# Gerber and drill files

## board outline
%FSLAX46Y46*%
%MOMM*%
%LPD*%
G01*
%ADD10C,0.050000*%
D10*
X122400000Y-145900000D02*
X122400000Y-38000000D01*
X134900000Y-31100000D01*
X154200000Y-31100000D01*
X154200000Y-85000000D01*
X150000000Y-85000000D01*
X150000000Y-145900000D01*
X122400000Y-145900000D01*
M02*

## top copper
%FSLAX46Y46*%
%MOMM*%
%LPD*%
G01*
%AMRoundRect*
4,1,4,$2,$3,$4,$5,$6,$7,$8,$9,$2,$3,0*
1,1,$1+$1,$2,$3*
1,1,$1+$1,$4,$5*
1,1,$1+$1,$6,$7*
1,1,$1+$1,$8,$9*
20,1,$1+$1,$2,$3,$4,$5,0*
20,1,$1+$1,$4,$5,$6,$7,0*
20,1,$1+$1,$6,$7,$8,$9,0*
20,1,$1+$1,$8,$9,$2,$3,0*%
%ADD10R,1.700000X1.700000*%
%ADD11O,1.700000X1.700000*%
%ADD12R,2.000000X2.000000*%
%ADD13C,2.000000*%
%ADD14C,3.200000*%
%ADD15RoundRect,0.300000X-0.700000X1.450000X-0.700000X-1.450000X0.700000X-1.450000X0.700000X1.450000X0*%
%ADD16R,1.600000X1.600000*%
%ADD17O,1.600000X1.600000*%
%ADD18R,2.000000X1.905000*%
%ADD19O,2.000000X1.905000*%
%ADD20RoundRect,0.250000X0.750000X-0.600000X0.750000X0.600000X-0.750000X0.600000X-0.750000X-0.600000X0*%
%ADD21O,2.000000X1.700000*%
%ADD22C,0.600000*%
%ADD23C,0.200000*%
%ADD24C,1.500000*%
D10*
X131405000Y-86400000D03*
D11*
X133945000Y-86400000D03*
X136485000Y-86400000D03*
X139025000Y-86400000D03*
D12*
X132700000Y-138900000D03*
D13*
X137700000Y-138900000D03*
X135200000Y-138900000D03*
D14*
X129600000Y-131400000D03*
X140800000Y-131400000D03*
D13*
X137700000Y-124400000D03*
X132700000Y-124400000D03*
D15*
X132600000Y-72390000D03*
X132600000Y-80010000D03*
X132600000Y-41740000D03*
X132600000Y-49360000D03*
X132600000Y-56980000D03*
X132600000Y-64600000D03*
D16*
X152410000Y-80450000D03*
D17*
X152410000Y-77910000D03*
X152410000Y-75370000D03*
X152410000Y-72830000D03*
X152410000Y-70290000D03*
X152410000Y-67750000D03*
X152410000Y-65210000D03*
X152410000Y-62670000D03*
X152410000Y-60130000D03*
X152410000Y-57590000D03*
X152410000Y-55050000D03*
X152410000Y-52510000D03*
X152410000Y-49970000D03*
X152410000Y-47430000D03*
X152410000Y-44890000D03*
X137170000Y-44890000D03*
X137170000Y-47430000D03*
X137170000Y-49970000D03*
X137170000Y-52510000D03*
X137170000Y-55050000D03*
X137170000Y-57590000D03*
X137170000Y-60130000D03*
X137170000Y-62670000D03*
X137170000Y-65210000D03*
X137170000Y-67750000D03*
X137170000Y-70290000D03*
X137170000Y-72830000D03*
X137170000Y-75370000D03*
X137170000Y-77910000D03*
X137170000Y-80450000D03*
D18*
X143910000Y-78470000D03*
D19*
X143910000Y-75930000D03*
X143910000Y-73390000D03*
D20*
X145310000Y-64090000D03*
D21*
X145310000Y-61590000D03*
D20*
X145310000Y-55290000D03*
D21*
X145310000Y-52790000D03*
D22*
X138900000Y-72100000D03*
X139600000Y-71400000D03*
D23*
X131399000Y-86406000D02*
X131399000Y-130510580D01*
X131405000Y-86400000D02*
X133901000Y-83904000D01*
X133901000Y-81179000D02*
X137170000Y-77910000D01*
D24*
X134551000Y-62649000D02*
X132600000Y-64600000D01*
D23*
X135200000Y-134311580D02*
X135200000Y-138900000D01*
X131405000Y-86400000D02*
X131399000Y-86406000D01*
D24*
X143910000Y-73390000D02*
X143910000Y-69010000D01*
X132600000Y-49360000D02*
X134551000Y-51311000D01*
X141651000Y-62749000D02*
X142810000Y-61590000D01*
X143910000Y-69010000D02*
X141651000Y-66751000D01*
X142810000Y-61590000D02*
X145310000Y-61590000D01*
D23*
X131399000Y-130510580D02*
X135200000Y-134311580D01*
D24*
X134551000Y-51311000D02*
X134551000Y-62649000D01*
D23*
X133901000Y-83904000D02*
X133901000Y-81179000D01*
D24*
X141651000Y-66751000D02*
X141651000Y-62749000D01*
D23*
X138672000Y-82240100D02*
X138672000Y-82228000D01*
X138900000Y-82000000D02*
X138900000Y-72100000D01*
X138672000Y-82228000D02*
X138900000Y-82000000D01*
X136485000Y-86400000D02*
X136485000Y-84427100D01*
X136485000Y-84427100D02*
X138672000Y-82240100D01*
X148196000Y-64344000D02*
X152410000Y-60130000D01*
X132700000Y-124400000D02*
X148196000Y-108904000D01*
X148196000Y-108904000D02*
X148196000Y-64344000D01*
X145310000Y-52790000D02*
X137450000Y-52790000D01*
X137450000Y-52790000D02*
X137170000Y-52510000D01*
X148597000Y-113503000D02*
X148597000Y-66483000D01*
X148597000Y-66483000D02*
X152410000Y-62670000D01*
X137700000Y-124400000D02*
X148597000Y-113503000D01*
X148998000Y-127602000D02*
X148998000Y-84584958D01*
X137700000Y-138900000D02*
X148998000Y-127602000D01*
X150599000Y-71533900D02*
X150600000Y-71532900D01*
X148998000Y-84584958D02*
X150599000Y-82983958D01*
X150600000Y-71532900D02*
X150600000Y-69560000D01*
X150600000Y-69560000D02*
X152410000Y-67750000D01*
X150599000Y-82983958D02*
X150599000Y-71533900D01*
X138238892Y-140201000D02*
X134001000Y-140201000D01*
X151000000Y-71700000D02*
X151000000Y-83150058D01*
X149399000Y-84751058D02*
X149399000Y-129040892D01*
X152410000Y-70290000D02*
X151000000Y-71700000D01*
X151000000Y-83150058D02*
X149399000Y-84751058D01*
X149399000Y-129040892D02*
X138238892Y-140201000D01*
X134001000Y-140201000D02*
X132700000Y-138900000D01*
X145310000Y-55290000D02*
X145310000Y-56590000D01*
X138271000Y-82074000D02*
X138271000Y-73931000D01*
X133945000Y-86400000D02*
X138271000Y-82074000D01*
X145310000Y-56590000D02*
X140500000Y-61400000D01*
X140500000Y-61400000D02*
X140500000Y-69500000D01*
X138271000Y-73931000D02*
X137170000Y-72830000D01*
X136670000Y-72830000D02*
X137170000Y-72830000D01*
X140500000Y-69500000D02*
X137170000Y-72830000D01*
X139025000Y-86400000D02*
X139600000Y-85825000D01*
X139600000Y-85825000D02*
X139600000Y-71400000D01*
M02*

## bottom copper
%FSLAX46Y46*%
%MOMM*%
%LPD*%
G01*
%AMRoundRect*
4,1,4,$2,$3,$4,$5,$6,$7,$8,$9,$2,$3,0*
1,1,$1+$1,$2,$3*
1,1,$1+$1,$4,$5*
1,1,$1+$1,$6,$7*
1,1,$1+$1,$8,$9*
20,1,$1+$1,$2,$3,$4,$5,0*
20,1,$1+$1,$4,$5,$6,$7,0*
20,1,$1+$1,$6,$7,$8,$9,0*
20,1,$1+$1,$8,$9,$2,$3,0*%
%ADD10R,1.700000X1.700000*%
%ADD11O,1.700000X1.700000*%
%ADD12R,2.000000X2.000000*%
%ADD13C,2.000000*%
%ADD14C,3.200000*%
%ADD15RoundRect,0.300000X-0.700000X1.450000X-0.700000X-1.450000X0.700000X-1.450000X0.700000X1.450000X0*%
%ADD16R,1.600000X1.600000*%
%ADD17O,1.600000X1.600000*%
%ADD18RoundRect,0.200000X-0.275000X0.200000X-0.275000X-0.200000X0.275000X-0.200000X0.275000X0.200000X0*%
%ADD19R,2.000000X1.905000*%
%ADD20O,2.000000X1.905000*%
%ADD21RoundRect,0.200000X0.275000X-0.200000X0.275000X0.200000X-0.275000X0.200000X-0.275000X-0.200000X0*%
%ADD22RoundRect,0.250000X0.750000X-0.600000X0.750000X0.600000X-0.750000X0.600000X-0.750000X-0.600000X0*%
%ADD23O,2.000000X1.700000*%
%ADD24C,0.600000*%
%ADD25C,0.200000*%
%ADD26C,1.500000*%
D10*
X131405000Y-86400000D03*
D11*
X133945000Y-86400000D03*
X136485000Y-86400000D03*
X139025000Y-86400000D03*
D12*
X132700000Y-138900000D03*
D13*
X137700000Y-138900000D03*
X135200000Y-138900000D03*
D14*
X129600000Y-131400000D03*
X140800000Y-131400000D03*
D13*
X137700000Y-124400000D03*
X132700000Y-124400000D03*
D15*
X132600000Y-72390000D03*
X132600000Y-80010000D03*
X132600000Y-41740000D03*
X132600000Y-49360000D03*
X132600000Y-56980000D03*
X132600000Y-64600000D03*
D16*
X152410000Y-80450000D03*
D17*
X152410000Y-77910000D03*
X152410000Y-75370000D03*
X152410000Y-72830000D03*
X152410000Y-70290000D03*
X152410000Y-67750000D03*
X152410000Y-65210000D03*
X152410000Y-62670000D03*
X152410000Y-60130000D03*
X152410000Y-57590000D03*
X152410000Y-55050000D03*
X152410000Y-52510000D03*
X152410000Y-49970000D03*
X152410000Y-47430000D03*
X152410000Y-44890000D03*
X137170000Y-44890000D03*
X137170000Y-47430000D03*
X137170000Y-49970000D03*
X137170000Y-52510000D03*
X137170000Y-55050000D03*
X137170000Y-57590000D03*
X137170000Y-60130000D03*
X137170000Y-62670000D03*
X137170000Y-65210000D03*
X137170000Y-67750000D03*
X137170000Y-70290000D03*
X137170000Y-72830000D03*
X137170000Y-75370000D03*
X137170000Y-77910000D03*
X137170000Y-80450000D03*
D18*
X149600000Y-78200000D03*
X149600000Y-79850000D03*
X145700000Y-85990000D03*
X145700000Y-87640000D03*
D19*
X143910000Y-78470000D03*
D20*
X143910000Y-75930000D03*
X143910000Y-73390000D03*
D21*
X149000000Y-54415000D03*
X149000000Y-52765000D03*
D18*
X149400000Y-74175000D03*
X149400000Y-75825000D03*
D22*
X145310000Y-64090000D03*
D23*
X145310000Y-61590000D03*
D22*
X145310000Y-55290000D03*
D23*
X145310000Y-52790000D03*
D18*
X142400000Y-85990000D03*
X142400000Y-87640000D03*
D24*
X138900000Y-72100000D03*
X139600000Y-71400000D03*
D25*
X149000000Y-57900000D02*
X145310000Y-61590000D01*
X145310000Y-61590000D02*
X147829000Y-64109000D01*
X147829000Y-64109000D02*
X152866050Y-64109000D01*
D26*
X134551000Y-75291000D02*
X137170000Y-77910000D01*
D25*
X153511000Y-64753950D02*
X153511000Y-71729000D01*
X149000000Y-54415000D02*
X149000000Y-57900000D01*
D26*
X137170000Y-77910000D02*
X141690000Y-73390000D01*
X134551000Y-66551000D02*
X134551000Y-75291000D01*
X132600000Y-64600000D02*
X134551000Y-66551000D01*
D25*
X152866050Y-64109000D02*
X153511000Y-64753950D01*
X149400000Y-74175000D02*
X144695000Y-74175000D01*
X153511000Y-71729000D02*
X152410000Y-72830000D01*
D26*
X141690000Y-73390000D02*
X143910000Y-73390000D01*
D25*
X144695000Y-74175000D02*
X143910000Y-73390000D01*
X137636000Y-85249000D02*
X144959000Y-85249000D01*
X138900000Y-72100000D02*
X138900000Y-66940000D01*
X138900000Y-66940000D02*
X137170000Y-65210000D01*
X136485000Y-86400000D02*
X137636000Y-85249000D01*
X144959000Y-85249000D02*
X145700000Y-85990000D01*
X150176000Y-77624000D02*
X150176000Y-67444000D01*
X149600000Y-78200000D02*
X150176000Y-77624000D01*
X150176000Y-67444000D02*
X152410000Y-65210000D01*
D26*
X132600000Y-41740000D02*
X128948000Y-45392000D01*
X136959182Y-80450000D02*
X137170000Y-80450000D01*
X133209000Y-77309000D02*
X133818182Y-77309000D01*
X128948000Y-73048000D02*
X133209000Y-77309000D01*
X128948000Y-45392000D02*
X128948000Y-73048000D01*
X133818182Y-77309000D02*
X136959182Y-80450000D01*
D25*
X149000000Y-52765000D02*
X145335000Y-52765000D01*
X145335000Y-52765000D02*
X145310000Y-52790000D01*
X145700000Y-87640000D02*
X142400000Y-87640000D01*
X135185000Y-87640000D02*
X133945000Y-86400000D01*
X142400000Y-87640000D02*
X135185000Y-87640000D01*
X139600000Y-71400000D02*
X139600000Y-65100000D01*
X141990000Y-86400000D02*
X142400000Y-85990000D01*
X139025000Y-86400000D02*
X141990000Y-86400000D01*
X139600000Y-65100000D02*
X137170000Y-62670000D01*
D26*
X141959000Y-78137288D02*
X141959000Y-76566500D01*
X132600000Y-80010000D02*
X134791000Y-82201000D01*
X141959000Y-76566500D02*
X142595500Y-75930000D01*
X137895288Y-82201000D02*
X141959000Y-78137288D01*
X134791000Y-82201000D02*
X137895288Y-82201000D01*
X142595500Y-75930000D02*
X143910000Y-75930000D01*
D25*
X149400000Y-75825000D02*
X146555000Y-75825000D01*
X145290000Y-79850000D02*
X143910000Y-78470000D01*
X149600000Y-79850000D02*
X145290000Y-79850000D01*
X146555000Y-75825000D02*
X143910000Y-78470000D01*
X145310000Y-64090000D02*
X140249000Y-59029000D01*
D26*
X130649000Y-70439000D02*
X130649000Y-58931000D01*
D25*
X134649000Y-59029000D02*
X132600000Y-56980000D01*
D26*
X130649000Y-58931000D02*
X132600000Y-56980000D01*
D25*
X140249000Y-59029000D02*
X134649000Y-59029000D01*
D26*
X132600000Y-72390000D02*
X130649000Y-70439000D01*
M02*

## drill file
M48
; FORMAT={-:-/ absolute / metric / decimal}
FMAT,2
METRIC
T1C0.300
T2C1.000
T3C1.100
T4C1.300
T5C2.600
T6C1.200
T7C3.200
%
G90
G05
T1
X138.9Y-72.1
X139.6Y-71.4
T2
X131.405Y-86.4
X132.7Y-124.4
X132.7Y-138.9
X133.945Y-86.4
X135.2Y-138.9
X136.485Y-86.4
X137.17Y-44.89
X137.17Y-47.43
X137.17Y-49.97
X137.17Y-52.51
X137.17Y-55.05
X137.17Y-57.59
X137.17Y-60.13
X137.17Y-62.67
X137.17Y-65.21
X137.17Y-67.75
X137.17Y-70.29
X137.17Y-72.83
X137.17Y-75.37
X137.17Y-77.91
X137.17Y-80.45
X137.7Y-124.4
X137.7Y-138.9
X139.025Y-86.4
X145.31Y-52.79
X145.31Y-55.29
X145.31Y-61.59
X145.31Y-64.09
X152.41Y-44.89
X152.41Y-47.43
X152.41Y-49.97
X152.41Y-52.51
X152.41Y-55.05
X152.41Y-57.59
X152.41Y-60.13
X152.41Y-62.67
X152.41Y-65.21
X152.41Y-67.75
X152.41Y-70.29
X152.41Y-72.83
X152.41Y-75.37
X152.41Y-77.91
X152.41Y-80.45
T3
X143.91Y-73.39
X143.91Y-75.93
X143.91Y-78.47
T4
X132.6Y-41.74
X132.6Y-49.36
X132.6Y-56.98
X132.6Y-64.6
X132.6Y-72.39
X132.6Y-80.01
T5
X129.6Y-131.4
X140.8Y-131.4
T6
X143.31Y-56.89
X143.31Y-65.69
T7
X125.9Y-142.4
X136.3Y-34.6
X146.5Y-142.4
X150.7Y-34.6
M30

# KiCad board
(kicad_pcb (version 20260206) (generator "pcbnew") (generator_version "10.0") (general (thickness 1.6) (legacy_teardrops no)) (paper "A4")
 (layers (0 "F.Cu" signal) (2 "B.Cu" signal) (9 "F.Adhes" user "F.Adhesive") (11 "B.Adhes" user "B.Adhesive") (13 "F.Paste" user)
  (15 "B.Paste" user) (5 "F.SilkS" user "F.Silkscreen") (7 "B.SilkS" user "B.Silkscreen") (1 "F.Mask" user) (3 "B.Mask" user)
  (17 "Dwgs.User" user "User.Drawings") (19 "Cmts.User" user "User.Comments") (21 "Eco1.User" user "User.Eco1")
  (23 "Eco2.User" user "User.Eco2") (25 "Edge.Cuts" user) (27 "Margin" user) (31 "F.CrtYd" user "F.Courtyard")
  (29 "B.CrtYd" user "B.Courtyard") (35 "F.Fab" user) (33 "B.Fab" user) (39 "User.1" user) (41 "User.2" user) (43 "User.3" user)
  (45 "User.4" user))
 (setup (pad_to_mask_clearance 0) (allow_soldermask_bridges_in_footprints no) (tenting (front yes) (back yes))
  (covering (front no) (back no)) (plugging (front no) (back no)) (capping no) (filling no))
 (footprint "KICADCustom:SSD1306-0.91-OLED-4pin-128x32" (layer "F.Cu") (at 129.215 122.9 90)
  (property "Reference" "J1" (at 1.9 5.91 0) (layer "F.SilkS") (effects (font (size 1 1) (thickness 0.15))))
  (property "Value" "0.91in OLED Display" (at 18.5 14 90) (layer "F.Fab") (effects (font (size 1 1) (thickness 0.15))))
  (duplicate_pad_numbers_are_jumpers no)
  (pad "1" thru_hole rect (at 36.5 2.19 90) (size 1.7 1.7) (drill 1) (layers "*.Cu" "*.Mask") (remove_unused_layers no) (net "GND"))
  (pad "2" thru_hole oval (at 36.5 4.73 90) (size 1.7 1.7) (drill 1) (layers "*.Cu" "*.Mask") (remove_unused_layers no) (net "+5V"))
  (pad "3" thru_hole oval (at 36.5 7.27 90) (size 1.7 1.7) (drill 1) (layers "*.Cu" "*.Mask") (remove_unused_layers no) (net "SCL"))
  (pad "4" thru_hole oval (at 36.5 9.81 90) (size 1.7 1.7) (drill 1) (layers "*.Cu" "*.Mask") (remove_unused_layers no) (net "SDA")))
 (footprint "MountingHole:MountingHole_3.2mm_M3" (layer "F.Cu") (at 146.5 142.4)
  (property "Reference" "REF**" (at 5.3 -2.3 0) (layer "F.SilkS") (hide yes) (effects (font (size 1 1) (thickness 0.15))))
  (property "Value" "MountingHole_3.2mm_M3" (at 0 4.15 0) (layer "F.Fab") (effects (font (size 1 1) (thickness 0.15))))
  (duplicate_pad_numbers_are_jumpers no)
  (pad "" np_thru_hole circle (at 0 0) (size 3.2 3.2) (drill 3.2) (layers "*.Cu" "*.Mask")))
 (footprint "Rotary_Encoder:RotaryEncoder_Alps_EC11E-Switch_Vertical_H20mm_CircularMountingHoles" (layer "F.Cu") (at 132.7 138.9 90)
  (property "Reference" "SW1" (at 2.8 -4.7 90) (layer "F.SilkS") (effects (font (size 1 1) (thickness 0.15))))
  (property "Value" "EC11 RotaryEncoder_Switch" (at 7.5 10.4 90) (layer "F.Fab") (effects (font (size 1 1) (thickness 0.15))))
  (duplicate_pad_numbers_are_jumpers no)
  (pad "A" thru_hole rect (at 0 0 90) (size 2 2) (drill 1) (layers "*.Cu" "*.Mask") (remove_unused_layers no) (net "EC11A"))
  (pad "B" thru_hole circle (at 0 5 90) (size 2 2) (drill 1) (layers "*.Cu" "*.Mask") (remove_unused_layers no) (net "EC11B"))
  (pad "C" thru_hole circle (at 0 2.5 90) (size 2 2) (drill 1) (layers "*.Cu" "*.Mask") (remove_unused_layers no) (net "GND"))
  (pad "MP" thru_hole circle (at 7.5 -3.1 90) (size 3.2 3.2) (drill 2.6) (layers "*.Cu" "*.Mask") (remove_unused_layers no))
  (pad "MP" thru_hole circle (at 7.5 8.1 90) (size 3.2 3.2) (drill 2.6) (layers "*.Cu" "*.Mask") (remove_unused_layers no))
  (pad "S1" thru_hole circle (at 14.5 5 90) (size 2 2) (drill 1) (layers "*.Cu" "*.Mask") (remove_unused_layers no) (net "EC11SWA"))
  (pad "S2" thru_hole circle (at 14.5 0 90) (size 2 2) (drill 1) (layers "*.Cu" "*.Mask") (remove_unused_layers no) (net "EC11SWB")))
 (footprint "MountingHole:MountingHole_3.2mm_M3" (layer "F.Cu") (at 136.3 34.6)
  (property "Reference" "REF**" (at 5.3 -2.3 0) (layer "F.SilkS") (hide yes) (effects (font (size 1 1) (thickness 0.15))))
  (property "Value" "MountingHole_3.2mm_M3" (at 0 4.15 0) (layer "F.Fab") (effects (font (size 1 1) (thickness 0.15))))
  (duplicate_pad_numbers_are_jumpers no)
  (pad "" np_thru_hole circle (at 0 0) (size 3.2 3.2) (drill 3.2) (layers "*.Cu" "*.Mask")))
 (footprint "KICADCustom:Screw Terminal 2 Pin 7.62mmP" (layer "F.Cu") (at 132.6 72.39 -90)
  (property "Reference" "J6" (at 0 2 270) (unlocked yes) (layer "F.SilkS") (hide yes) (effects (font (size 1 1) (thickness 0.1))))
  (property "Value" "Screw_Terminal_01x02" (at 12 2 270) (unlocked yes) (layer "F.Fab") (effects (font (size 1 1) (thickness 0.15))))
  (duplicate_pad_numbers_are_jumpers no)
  (pad "1" thru_hole roundrect (at 0 0 270) (size 3.5 2) (drill 1.3) (layers "*.Cu" "*.Mask") (remove_unused_layers no)
   (roundrect_rratio 0.15) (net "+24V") (thermal_bridge_angle 45))
  (pad "2" thru_hole roundrect (at 7.62 0 270) (size 3.5 2) (drill 1.3) (layers "*.Cu" "*.Mask") (remove_unused_layers no)
   (roundrect_rratio 0.15) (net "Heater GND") (thermal_bridge_angle 45)))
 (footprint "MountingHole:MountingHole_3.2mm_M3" (layer "F.Cu") (at 150.7 34.6)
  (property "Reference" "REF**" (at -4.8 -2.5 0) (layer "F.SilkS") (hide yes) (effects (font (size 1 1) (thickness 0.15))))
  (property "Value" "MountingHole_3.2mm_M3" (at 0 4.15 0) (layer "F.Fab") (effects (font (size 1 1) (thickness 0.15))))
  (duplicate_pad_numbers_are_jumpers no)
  (pad "" np_thru_hole circle (at 0 0) (size 3.2 3.2) (drill 3.2) (layers "*.Cu" "*.Mask")))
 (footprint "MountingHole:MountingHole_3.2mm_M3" (layer "F.Cu") (at 125.9 142.4)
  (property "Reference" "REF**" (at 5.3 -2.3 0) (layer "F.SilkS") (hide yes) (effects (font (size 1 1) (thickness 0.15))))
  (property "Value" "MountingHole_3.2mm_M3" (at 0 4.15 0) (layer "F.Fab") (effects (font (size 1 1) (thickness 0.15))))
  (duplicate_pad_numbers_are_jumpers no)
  (pad "" np_thru_hole circle (at 0 0) (size 3.2 3.2) (drill 3.2) (layers "*.Cu" "*.Mask")))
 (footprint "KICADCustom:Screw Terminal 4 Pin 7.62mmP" (layer "F.Cu") (at 132.6 41.74 -90)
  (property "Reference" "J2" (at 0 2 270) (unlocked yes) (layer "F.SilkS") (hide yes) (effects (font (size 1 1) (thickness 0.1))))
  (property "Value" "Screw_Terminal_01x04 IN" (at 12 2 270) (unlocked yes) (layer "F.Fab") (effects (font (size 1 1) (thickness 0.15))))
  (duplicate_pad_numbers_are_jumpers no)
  (pad "1" thru_hole roundrect (at 0 0 270) (size 3.5 2) (drill 1.3) (layers "*.Cu" "*.Mask") (remove_unused_layers no)
   (roundrect_rratio 0.15) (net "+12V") (thermal_bridge_angle 45))
  (pad "2" thru_hole roundrect (at 7.62 0 270) (size 3.5 2) (drill 1.3) (layers "*.Cu" "*.Mask") (remove_unused_layers no)
   (roundrect_rratio 0.15) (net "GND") (thermal_bridge_angle 45))
  (pad "3" thru_hole roundrect (at 15.24 0 270) (size 3.5 2) (drill 1.3) (layers "*.Cu" "*.Mask") (remove_unused_layers no)
   (roundrect_rratio 0.15) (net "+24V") (thermal_bridge_angle 45))
  (pad "4" thru_hole roundrect (at 22.86 0 270) (size 3.5 2) (drill 1.3) (layers "*.Cu" "*.Mask") (remove_unused_layers no)
   (roundrect_rratio 0.15) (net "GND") (thermal_bridge_angle 45)))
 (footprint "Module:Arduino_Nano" (layer "F.Cu") (at 152.41 80.45 180)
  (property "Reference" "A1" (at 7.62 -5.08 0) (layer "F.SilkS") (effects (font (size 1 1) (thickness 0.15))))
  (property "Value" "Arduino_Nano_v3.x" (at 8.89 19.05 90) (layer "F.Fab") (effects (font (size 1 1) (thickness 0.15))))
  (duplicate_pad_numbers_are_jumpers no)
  (pad "1" thru_hole rect (at 0 0 180) (size 1.6 1.6) (drill 1) (layers "*.Cu" "*.Mask") (remove_unused_layers no)
   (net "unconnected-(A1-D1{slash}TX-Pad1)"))
  (pad "2" thru_hole oval (at 0 2.54 180) (size 1.6 1.6) (drill 1) (layers "*.Cu" "*.Mask") (remove_unused_layers no)
   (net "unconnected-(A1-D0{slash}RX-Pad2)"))
  (pad "3" thru_hole oval (at 0 5.08 180) (size 1.6 1.6) (drill 1) (layers "*.Cu" "*.Mask") (remove_unused_layers no)
   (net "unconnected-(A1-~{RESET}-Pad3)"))
  (pad "4" thru_hole oval (at 0 7.62 180) (size 1.6 1.6) (drill 1) (layers "*.Cu" "*.Mask") (remove_unused_layers no) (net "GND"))
  (pad "5" thru_hole oval (at 0 10.16 180) (size 1.6 1.6) (drill 1) (layers "*.Cu" "*.Mask") (remove_unused_layers no) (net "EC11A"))
  (pad "6" thru_hole oval (at 0 12.7 180) (size 1.6 1.6) (drill 1) (layers "*.Cu" "*.Mask") (remove_unused_layers no) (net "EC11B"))
  (pad "7" thru_hole oval (at 0 15.24 180) (size 1.6 1.6) (drill 1) (layers "*.Cu" "*.Mask") (remove_unused_layers no) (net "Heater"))
  (pad "8" thru_hole oval (at 0 17.78 180) (size 1.6 1.6) (drill 1) (layers "*.Cu" "*.Mask") (remove_unused_layers no) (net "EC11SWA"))
  (pad "9" thru_hole oval (at 0 20.32 180) (size 1.6 1.6) (drill 1) (layers "*.Cu" "*.Mask") (remove_unused_layers no) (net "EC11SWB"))
  (pad "10" thru_hole oval (at 0 22.86 180) (size 1.6 1.6) (drill 1) (layers "*.Cu" "*.Mask") (remove_unused_layers no)
   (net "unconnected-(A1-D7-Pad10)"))
  (pad "11" thru_hole oval (at 0 25.4 180) (size 1.6 1.6) (drill 1) (layers "*.Cu" "*.Mask") (remove_unused_layers no)
   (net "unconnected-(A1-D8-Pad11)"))
  (pad "12" thru_hole oval (at 0 27.94 180) (size 1.6 1.6) (drill 1) (layers "*.Cu" "*.Mask") (remove_unused_layers no)
   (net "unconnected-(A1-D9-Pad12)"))
  (pad "13" thru_hole oval (at 0 30.48 180) (size 1.6 1.6) (drill 1) (layers "*.Cu" "*.Mask") (remove_unused_layers no)
   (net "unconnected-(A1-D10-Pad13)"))
  (pad "14" thru_hole oval (at 0 33.02 180) (size 1.6 1.6) (drill 1) (layers "*.Cu" "*.Mask") (remove_unused_layers no)
   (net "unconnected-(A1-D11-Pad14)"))
  (pad "15" thru_hole oval (at 0 35.56 180) (size 1.6 1.6) (drill 1) (layers "*.Cu" "*.Mask") (remove_unused_layers no)
   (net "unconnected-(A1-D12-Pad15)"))
  (pad "16" thru_hole oval (at 15.24 35.56 180) (size 1.6 1.6) (drill 1) (layers "*.Cu" "*.Mask") (remove_unused_layers no)
   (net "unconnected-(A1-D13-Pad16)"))
  (pad "17" thru_hole oval (at 15.24 33.02 180) (size 1.6 1.6) (drill 1) (layers "*.Cu" "*.Mask") (remove_unused_layers no)
   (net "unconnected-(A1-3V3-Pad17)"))
  (pad "18" thru_hole oval (at 15.24 30.48 180) (size 1.6 1.6) (drill 1) (layers "*.Cu" "*.Mask") (remove_unused_layers no)
   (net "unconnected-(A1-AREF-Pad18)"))
  (pad "19" thru_hole oval (at 15.24 27.94 180) (size 1.6 1.6) (drill 1) (layers "*.Cu" "*.Mask") (remove_unused_layers no)
   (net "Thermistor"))
  (pad "20" thru_hole oval (at 15.24 25.4 180) (size 1.6 1.6) (drill 1) (layers "*.Cu" "*.Mask") (remove_unused_layers no)
   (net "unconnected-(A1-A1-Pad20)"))
  (pad "21" thru_hole oval (at 15.24 22.86 180) (size 1.6 1.6) (drill 1) (layers "*.Cu" "*.Mask") (remove_unused_layers no)
   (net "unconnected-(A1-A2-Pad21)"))
  (pad "22" thru_hole oval (at 15.24 20.32 180) (size 1.6 1.6) (drill 1) (layers "*.Cu" "*.Mask") (remove_unused_layers no)
   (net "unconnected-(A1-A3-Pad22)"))
  (pad "23" thru_hole oval (at 15.24 17.78 180) (size 1.6 1.6) (drill 1) (layers "*.Cu" "*.Mask") (remove_unused_layers no) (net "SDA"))
  (pad "24" thru_hole oval (at 15.24 15.24 180) (size 1.6 1.6) (drill 1) (layers "*.Cu" "*.Mask") (remove_unused_layers no) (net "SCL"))
  (pad "25" thru_hole oval (at 15.24 12.7 180) (size 1.6 1.6) (drill 1) (layers "*.Cu" "*.Mask") (remove_unused_layers no)
   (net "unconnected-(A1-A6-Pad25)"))
  (pad "26" thru_hole oval (at 15.24 10.16 180) (size 1.6 1.6) (drill 1) (layers "*.Cu" "*.Mask") (remove_unused_layers no)
   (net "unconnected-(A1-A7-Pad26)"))
  (pad "27" thru_hole oval (at 15.24 7.62 180) (size 1.6 1.6) (drill 1) (layers "*.Cu" "*.Mask") (remove_unused_layers no) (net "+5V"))
  (pad "28" thru_hole oval (at 15.24 5.08 180) (size 1.6 1.6) (drill 1) (layers "*.Cu" "*.Mask") (remove_unused_layers no)
   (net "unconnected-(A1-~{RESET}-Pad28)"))
  (pad "29" thru_hole oval (at 15.24 2.54 180) (size 1.6 1.6) (drill 1) (layers "*.Cu" "*.Mask") (remove_unused_layers no) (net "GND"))
  (pad "30" thru_hole oval (at 15.24 0 180) (size 1.6 1.6) (drill 1) (layers "*.Cu" "*.Mask") (remove_unused_layers no) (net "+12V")))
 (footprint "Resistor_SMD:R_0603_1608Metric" (layer "B.Cu") (at 149.6 79.025 -90)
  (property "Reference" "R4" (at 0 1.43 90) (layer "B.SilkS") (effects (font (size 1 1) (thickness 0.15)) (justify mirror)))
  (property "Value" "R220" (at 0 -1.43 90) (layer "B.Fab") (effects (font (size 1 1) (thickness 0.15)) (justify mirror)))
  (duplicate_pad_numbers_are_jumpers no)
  (pad "1" smd roundrect (at -0.825 0 270) (size 0.8 0.95) (layers "B.Cu" "B.Mask" "B.Paste") (roundrect_rratio 0.25) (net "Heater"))
  (pad "2" smd roundrect (at 0.825 0 270) (size 0.8 0.95) (layers "B.Cu" "B.Mask" "B.Paste") (roundrect_rratio 0.25) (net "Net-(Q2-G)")))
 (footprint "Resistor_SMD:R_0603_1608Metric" (layer "B.Cu") (at 145.7 86.815 -90)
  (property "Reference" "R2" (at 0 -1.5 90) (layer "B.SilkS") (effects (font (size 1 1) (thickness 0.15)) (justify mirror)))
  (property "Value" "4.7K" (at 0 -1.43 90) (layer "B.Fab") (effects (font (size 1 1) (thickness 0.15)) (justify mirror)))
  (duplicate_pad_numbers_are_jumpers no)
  (pad "1" smd roundrect (at -0.825 0 270) (size 0.8 0.95) (layers "B.Cu" "B.Mask" "B.Paste") (roundrect_rratio 0.25) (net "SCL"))
  (pad "2" smd roundrect (at 0.825 0 270) (size 0.8 0.95) (layers "B.Cu" "B.Mask" "B.Paste") (roundrect_rratio 0.25) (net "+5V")))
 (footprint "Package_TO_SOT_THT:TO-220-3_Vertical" (layer "B.Cu") (at 143.91 78.47 90)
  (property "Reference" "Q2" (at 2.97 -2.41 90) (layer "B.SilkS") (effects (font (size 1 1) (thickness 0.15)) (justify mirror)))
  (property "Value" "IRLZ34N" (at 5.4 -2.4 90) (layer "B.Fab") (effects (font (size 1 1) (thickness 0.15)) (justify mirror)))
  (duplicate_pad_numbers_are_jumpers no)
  (pad "1" thru_hole rect (at 0 0 90) (size 1.905 2) (drill 1.1) (layers "*.Cu" "*.Mask") (remove_unused_layers no) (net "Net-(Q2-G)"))
  (pad "2" thru_hole oval (at 2.54 0 90) (size 1.905 2) (drill 1.1) (layers "*.Cu" "*.Mask") (remove_unused_layers no) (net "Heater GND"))
  (pad "3" thru_hole oval (at 5.08 0 90) (size 1.905 2) (drill 1.1) (layers "*.Cu" "*.Mask") (remove_unused_layers no) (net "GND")))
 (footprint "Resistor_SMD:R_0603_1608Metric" (layer "B.Cu") (at 149 53.59 90)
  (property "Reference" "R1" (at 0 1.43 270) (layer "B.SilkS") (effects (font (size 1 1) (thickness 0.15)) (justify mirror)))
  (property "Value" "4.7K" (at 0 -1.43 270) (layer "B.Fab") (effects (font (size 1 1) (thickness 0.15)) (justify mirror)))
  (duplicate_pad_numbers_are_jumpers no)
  (pad "1" smd roundrect (at -0.825 0 90) (size 0.8 0.95) (layers "B.Cu" "B.Mask" "B.Paste") (roundrect_rratio 0.25) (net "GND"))
  (pad "2" smd roundrect (at 0.825 0 90) (size 0.8 0.95) (layers "B.Cu" "B.Mask" "B.Paste") (roundrect_rratio 0.25) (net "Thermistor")))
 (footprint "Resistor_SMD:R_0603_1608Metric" (layer "B.Cu") (at 149.4 75 -90)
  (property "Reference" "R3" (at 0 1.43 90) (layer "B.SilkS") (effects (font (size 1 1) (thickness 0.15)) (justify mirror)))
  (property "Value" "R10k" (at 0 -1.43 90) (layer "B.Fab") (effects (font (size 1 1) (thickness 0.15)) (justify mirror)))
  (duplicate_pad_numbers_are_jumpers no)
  (pad "1" smd roundrect (at -0.825 0 270) (size 0.8 0.95) (layers "B.Cu" "B.Mask" "B.Paste") (roundrect_rratio 0.25) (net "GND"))
  (pad "2" smd roundrect (at 0.825 0 270) (size 0.8 0.95) (layers "B.Cu" "B.Mask" "B.Paste") (roundrect_rratio 0.25) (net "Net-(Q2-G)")))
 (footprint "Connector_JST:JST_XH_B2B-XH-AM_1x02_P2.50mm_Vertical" (layer "B.Cu") (at 145.31 64.09 90)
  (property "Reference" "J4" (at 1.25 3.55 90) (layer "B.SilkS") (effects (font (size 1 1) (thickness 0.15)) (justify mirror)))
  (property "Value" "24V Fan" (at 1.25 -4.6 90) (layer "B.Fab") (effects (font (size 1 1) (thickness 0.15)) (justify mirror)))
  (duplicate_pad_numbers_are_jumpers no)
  (pad "" np_thru_hole circle (at -1.6 -2 90) (size 1.2 1.2) (drill 1.2) (layers "*.Cu" "*.Mask"))
  (pad "1" thru_hole roundrect (at 0 0 90) (size 1.7 2) (drill 1) (layers "*.Cu" "*.Mask") (remove_unused_layers no)
   (roundrect_rratio 0.147059) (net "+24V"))
  (pad "2" thru_hole oval (at 2.5 0 90) (size 1.7 2) (drill 1) (layers "*.Cu" "*.Mask") (remove_unused_layers no) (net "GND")))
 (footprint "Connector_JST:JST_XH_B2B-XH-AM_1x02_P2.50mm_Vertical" (layer "B.Cu") (at 145.31 55.29 90)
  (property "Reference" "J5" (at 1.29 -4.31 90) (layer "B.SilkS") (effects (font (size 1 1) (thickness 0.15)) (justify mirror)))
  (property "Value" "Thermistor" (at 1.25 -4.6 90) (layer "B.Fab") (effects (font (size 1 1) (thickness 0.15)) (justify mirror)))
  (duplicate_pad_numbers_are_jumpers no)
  (pad "" np_thru_hole circle (at -1.6 -2 90) (size 1.2 1.2) (drill 1.2) (layers "*.Cu" "*.Mask"))
  (pad "1" thru_hole roundrect (at 0 0 90) (size 1.7 2) (drill 1) (layers "*.Cu" "*.Mask") (remove_unused_layers no)
   (roundrect_rratio 0.147059) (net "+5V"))
  (pad "2" thru_hole oval (at 2.5 0 90) (size 1.7 2) (drill 1) (layers "*.Cu" "*.Mask") (remove_unused_layers no) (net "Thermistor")))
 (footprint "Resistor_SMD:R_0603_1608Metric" (layer "B.Cu") (at 142.4 86.815 -90)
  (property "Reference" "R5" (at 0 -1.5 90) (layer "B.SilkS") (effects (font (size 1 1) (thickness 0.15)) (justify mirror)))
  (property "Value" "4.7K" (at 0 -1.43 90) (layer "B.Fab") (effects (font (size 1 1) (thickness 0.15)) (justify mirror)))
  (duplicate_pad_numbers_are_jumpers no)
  (pad "1" smd roundrect (at -0.825 0 270) (size 0.8 0.95) (layers "B.Cu" "B.Mask" "B.Paste") (roundrect_rratio 0.25) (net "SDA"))
  (pad "2" smd roundrect (at 0.825 0 270) (size 0.8 0.95) (layers "B.Cu" "B.Mask" "B.Paste") (roundrect_rratio 0.25) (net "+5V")))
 (gr_poly
  (pts (xy 122.4 145.9) (xy 122.4 38) (xy 134.9 31.1) (xy 154.2 31.1) (xy 154.2 85) (xy 150 85) (xy 150 145.9))
  (stroke (width 0.05) (type solid)) (fill no) (layer "Edge.Cuts"))
 (segment (start 131.399 86.406) (end 131.399 130.51058) (width 0.2) (layer "F.Cu") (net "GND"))
 (segment (start 131.405 86.4) (end 133.901 83.904) (width 0.2) (layer "F.Cu") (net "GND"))
 (segment (start 133.901 81.179) (end 137.17 77.91) (width 0.2) (layer "F.Cu") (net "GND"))
 (segment (start 134.551 62.649) (end 132.6 64.6) (width 1.5) (layer "F.Cu") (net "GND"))
 (segment (start 135.2 134.31158) (end 135.2 138.9) (width 0.2) (layer "F.Cu") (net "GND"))
 (segment (start 131.405 86.4) (end 131.399 86.406) (width 0.2) (layer "F.Cu") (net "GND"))
 (segment (start 143.91 73.39) (end 143.91 69.01) (width 1.5) (layer "F.Cu") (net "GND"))
 (segment (start 132.6 49.36) (end 134.551 51.311) (width 1.5) (layer "F.Cu") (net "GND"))
 (segment (start 141.651 62.749) (end 142.81 61.59) (width 1.5) (layer "F.Cu") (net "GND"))
 (segment (start 143.91 69.01) (end 141.651 66.751) (width 1.5) (layer "F.Cu") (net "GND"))
 (segment (start 142.81 61.59) (end 145.31 61.59) (width 1.5) (layer "F.Cu") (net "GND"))
 (segment (start 131.399 130.51058) (end 135.2 134.31158) (width 0.2) (layer "F.Cu") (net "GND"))
 (segment (start 134.551 51.311) (end 134.551 62.649) (width 1.5) (layer "F.Cu") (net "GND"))
 (segment (start 133.901 83.904) (end 133.901 81.179) (width 0.2) (layer "F.Cu") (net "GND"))
 (segment (start 141.651 66.751) (end 141.651 62.749) (width 1.5) (layer "F.Cu") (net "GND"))
 (segment (start 149 57.9) (end 145.31 61.59) (width 0.2) (layer "B.Cu") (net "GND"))
 (segment (start 145.31 61.59) (end 147.829 64.109) (width 0.2) (layer "B.Cu") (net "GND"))
 (segment (start 147.829 64.109) (end 152.86605 64.109) (width 0.2) (layer "B.Cu") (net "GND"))
 (segment (start 134.551 75.291) (end 137.17 77.91) (width 1.5) (layer "B.Cu") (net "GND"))
 (segment (start 153.511 64.75395) (end 153.511 71.729) (width 0.2) (layer "B.Cu") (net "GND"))
 (segment (start 149 54.415) (end 149 57.9) (width 0.2) (layer "B.Cu") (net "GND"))
 (segment (start 137.17 77.91) (end 141.69 73.39) (width 1.5) (layer "B.Cu") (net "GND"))
 (segment (start 134.551 66.551) (end 134.551 75.291) (width 1.5) (layer "B.Cu") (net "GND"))
 (segment (start 132.6 64.6) (end 134.551 66.551) (width 1.5) (layer "B.Cu") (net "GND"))
 (segment (start 152.86605 64.109) (end 153.511 64.75395) (width 0.2) (layer "B.Cu") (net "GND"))
 (segment (start 149.4 74.175) (end 144.695 74.175) (width 0.2) (layer "B.Cu") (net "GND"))
 (segment (start 153.511 71.729) (end 152.41 72.83) (width 0.2) (layer "B.Cu") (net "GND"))
 (segment (start 141.69 73.39) (end 143.91 73.39) (width 1.5) (layer "B.Cu") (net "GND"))
 (segment (start 144.695 74.175) (end 143.91 73.39) (width 0.2) (layer "B.Cu") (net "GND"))
 (segment (start 138.672 82.2401) (end 138.672 82.228) (width 0.2) (layer "F.Cu") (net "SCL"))
 (segment (start 138.9 82) (end 138.9 72.1) (width 0.2) (layer "F.Cu") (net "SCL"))
 (segment (start 138.672 82.228) (end 138.9 82) (width 0.2) (layer "F.Cu") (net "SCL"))
 (segment (start 136.485 86.4) (end 136.485 84.4271) (width 0.2) (layer "F.Cu") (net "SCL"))
 (segment (start 136.485 84.4271) (end 138.672 82.2401) (width 0.2) (layer "F.Cu") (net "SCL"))
 (via (at 138.9 72.1) (size 0.6) (drill 0.3) (layers "F.Cu" "B.Cu") (capping no) (covering (front no) (back no))
  (plugging (front no) (back no)) (filling no) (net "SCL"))
 (segment (start 137.636 85.249) (end 144.959 85.249) (width 0.2) (layer "B.Cu") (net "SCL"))
 (segment (start 138.9 72.1) (end 138.9 66.94) (width 0.2) (layer "B.Cu") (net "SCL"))
 (segment (start 138.9 66.94) (end 137.17 65.21) (width 0.2) (layer "B.Cu") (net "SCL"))
 (segment (start 136.485 86.4) (end 137.636 85.249) (width 0.2) (layer "B.Cu") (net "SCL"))
 (segment (start 144.959 85.249) (end 145.7 85.99) (width 0.2) (layer "B.Cu") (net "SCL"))
 (segment (start 150.176 77.624) (end 150.176 67.444) (width 0.2) (layer "B.Cu") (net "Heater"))
 (segment (start 149.6 78.2) (end 150.176 77.624) (width 0.2) (layer "B.Cu") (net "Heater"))
 (segment (start 150.176 67.444) (end 152.41 65.21) (width 0.2) (layer "B.Cu") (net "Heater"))
 (segment (start 148.196 64.344) (end 152.41 60.13) (width 0.2) (layer "F.Cu") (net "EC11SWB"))
 (segment (start 132.7 124.4) (end 148.196 108.904) (width 0.2) (layer "F.Cu") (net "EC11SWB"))
 (segment (start 148.196 108.904) (end 148.196 64.344) (width 0.2) (layer "F.Cu") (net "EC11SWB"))
 (segment (start 132.6 41.74) (end 128.948 45.392) (width 1.5) (layer "B.Cu") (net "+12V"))
 (segment (start 136.959182 80.45) (end 137.17 80.45) (width 1.5) (layer "B.Cu") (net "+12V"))
 (segment (start 133.209 77.309) (end 133.818182 77.309) (width 1.5) (layer "B.Cu") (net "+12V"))
 (segment (start 128.948 73.048) (end 133.209 77.309) (width 1.5) (layer "B.Cu") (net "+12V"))
 (segment (start 128.948 45.392) (end 128.948 73.048) (width 1.5) (layer "B.Cu") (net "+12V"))
 (segment (start 133.818182 77.309) (end 136.959182 80.45) (width 1.5) (layer "B.Cu") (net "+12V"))
 (segment (start 145.31 52.79) (end 137.45 52.79) (width 0.2) (layer "F.Cu") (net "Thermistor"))
 (segment (start 137.45 52.79) (end 137.17 52.51) (width 0.2) (layer "F.Cu") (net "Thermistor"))
 (segment (start 149 52.765) (end 145.335 52.765) (width 0.2) (layer "B.Cu") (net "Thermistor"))
 (segment (start 145.335 52.765) (end 145.31 52.79) (width 0.2) (layer "B.Cu") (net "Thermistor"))
 (segment (start 148.597 113.503) (end 148.597 66.483) (width 0.2) (layer "F.Cu") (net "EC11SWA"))
 (segment (start 148.597 66.483) (end 152.41 62.67) (width 0.2) (layer "F.Cu") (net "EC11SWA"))
 (segment (start 137.7 124.4) (end 148.597 113.503) (width 0.2) (layer "F.Cu") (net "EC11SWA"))
 (segment (start 148.998 127.602) (end 148.998 84.584958) (width 0.2) (layer "F.Cu") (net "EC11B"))
 (segment (start 137.7 138.9) (end 148.998 127.602) (width 0.2) (layer "F.Cu") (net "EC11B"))
 (segment (start 150.599 71.5339) (end 150.6 71.5329) (width 0.2) (layer "F.Cu") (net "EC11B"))
 (segment (start 148.998 84.584958) (end 150.599 82.983958) (width 0.2) (layer "F.Cu") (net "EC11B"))
 (segment (start 150.6 71.5329) (end 150.6 69.56) (width 0.2) (layer "F.Cu") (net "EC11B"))
 (segment (start 150.6 69.56) (end 152.41 67.75) (width 0.2) (layer "F.Cu") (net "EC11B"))
 (segment (start 150.599 82.983958) (end 150.599 71.5339) (width 0.2) (layer "F.Cu") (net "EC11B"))
 (segment (start 138.238892 140.201) (end 134.001 140.201) (width 0.2) (layer "F.Cu") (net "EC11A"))
 (segment (start 151 71.7) (end 151 83.150058) (width 0.2) (layer "F.Cu") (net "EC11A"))
 (segment (start 149.399 84.751058) (end 149.399 129.040892) (width 0.2) (layer "F.Cu") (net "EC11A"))
 (segment (start 152.41 70.29) (end 151 71.7) (width 0.2) (layer "F.Cu") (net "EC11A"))
 (segment (start 151 83.150058) (end 149.399 84.751058) (width 0.2) (layer "F.Cu") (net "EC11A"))
 (segment (start 149.399 129.040892) (end 138.238892 140.201) (width 0.2) (layer "F.Cu") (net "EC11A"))
 (segment (start 134.001 140.201) (end 132.7 138.9) (width 0.2) (layer "F.Cu") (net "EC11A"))
 (segment (start 145.31 55.29) (end 145.31 56.59) (width 0.2) (layer "F.Cu") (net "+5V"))
 (segment (start 138.271 82.074) (end 138.271 73.931) (width 0.2) (layer "F.Cu") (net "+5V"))
 (segment (start 133.945 86.4) (end 138.271 82.074) (width 0.2) (layer "F.Cu") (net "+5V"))
 (segment (start 145.31 56.59) (end 140.5 61.4) (width 0.2) (layer "F.Cu") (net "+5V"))
 (segment (start 140.5 61.4) (end 140.5 69.5) (width 0.2) (layer "F.Cu") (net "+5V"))
 (segment (start 138.271 73.931) (end 137.17 72.83) (width 0.2) (layer "F.Cu") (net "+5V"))
 (segment (start 136.67 72.83) (end 137.17 72.83) (width 0.2) (layer "F.Cu") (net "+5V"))
 (segment (start 140.5 69.5) (end 137.17 72.83) (width 0.2) (layer "F.Cu") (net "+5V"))
 (segment (start 145.7 87.64) (end 142.4 87.64) (width 0.2) (layer "B.Cu") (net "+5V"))
 (segment (start 135.185 87.64) (end 133.945 86.4) (width 0.2) (layer "B.Cu") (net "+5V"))
 (segment (start 142.4 87.64) (end 135.185 87.64) (width 0.2) (layer "B.Cu") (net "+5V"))
 (segment (start 139.025 86.4) (end 139.6 85.825) (width 0.2) (layer "F.Cu") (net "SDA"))
 (segment (start 139.6 85.825) (end 139.6 71.4) (width 0.2) (layer "F.Cu") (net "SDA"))
 (via (at 139.6 71.4) (size 0.6) (drill 0.3) (layers "F.Cu" "B.Cu") (capping no) (covering (front no) (back no))
  (plugging (front no) (back no)) (filling no) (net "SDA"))
 (segment (start 139.6 71.4) (end 139.6 65.1) (width 0.2) (layer "B.Cu") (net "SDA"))
 (segment (start 141.99 86.4) (end 142.4 85.99) (width 0.2) (layer "B.Cu") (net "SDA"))
 (segment (start 139.025 86.4) (end 141.99 86.4) (width 0.2) (layer "B.Cu") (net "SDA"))
 (segment (start 139.6 65.1) (end 137.17 62.67) (width 0.2) (layer "B.Cu") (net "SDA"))
 (segment (start 141.959 78.137288) (end 141.959 76.5665) (width 1.5) (layer "B.Cu") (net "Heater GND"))
 (segment (start 132.6 80.01) (end 134.791 82.201) (width 1.5) (layer "B.Cu") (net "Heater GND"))
 (segment (start 141.959 76.5665) (end 142.5955 75.93) (width 1.5) (layer "B.Cu") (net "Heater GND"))
 (segment (start 137.895288 82.201) (end 141.959 78.137288) (width 1.5) (layer "B.Cu") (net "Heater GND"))
 (segment (start 134.791 82.201) (end 137.895288 82.201) (width 1.5) (layer "B.Cu") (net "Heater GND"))
 (segment (start 142.5955 75.93) (end 143.91 75.93) (width 1.5) (layer "B.Cu") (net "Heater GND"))
 (segment (start 149.4 75.825) (end 146.555 75.825) (width 0.2) (layer "B.Cu") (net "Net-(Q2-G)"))
 (segment (start 145.29 79.85) (end 143.91 78.47) (width 0.2) (layer "B.Cu") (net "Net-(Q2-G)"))
 (segment (start 149.6 79.85) (end 145.29 79.85) (width 0.2) (layer "B.Cu") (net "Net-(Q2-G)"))
 (segment (start 146.555 75.825) (end 143.91 78.47) (width 0.2) (layer "B.Cu") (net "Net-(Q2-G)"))
 (segment (start 145.31 64.09) (end 140.249 59.029) (width 0.2) (layer "B.Cu") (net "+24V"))
 (segment (start 130.649 70.439) (end 130.649 58.931) (width 1.5) (layer "B.Cu") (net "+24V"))
 (segment (start 134.649 59.029) (end 132.6 56.98) (width 0.2) (layer "B.Cu") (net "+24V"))
 (segment (start 130.649 58.931) (end 132.6 56.98) (width 1.5) (layer "B.Cu") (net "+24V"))
 (segment (start 140.249 59.029) (end 134.649 59.029) (width 0.2) (layer "B.Cu") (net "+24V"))
 (segment (start 132.6 72.39) (end 130.649 70.439) (width 1.5) (layer "B.Cu") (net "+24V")))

